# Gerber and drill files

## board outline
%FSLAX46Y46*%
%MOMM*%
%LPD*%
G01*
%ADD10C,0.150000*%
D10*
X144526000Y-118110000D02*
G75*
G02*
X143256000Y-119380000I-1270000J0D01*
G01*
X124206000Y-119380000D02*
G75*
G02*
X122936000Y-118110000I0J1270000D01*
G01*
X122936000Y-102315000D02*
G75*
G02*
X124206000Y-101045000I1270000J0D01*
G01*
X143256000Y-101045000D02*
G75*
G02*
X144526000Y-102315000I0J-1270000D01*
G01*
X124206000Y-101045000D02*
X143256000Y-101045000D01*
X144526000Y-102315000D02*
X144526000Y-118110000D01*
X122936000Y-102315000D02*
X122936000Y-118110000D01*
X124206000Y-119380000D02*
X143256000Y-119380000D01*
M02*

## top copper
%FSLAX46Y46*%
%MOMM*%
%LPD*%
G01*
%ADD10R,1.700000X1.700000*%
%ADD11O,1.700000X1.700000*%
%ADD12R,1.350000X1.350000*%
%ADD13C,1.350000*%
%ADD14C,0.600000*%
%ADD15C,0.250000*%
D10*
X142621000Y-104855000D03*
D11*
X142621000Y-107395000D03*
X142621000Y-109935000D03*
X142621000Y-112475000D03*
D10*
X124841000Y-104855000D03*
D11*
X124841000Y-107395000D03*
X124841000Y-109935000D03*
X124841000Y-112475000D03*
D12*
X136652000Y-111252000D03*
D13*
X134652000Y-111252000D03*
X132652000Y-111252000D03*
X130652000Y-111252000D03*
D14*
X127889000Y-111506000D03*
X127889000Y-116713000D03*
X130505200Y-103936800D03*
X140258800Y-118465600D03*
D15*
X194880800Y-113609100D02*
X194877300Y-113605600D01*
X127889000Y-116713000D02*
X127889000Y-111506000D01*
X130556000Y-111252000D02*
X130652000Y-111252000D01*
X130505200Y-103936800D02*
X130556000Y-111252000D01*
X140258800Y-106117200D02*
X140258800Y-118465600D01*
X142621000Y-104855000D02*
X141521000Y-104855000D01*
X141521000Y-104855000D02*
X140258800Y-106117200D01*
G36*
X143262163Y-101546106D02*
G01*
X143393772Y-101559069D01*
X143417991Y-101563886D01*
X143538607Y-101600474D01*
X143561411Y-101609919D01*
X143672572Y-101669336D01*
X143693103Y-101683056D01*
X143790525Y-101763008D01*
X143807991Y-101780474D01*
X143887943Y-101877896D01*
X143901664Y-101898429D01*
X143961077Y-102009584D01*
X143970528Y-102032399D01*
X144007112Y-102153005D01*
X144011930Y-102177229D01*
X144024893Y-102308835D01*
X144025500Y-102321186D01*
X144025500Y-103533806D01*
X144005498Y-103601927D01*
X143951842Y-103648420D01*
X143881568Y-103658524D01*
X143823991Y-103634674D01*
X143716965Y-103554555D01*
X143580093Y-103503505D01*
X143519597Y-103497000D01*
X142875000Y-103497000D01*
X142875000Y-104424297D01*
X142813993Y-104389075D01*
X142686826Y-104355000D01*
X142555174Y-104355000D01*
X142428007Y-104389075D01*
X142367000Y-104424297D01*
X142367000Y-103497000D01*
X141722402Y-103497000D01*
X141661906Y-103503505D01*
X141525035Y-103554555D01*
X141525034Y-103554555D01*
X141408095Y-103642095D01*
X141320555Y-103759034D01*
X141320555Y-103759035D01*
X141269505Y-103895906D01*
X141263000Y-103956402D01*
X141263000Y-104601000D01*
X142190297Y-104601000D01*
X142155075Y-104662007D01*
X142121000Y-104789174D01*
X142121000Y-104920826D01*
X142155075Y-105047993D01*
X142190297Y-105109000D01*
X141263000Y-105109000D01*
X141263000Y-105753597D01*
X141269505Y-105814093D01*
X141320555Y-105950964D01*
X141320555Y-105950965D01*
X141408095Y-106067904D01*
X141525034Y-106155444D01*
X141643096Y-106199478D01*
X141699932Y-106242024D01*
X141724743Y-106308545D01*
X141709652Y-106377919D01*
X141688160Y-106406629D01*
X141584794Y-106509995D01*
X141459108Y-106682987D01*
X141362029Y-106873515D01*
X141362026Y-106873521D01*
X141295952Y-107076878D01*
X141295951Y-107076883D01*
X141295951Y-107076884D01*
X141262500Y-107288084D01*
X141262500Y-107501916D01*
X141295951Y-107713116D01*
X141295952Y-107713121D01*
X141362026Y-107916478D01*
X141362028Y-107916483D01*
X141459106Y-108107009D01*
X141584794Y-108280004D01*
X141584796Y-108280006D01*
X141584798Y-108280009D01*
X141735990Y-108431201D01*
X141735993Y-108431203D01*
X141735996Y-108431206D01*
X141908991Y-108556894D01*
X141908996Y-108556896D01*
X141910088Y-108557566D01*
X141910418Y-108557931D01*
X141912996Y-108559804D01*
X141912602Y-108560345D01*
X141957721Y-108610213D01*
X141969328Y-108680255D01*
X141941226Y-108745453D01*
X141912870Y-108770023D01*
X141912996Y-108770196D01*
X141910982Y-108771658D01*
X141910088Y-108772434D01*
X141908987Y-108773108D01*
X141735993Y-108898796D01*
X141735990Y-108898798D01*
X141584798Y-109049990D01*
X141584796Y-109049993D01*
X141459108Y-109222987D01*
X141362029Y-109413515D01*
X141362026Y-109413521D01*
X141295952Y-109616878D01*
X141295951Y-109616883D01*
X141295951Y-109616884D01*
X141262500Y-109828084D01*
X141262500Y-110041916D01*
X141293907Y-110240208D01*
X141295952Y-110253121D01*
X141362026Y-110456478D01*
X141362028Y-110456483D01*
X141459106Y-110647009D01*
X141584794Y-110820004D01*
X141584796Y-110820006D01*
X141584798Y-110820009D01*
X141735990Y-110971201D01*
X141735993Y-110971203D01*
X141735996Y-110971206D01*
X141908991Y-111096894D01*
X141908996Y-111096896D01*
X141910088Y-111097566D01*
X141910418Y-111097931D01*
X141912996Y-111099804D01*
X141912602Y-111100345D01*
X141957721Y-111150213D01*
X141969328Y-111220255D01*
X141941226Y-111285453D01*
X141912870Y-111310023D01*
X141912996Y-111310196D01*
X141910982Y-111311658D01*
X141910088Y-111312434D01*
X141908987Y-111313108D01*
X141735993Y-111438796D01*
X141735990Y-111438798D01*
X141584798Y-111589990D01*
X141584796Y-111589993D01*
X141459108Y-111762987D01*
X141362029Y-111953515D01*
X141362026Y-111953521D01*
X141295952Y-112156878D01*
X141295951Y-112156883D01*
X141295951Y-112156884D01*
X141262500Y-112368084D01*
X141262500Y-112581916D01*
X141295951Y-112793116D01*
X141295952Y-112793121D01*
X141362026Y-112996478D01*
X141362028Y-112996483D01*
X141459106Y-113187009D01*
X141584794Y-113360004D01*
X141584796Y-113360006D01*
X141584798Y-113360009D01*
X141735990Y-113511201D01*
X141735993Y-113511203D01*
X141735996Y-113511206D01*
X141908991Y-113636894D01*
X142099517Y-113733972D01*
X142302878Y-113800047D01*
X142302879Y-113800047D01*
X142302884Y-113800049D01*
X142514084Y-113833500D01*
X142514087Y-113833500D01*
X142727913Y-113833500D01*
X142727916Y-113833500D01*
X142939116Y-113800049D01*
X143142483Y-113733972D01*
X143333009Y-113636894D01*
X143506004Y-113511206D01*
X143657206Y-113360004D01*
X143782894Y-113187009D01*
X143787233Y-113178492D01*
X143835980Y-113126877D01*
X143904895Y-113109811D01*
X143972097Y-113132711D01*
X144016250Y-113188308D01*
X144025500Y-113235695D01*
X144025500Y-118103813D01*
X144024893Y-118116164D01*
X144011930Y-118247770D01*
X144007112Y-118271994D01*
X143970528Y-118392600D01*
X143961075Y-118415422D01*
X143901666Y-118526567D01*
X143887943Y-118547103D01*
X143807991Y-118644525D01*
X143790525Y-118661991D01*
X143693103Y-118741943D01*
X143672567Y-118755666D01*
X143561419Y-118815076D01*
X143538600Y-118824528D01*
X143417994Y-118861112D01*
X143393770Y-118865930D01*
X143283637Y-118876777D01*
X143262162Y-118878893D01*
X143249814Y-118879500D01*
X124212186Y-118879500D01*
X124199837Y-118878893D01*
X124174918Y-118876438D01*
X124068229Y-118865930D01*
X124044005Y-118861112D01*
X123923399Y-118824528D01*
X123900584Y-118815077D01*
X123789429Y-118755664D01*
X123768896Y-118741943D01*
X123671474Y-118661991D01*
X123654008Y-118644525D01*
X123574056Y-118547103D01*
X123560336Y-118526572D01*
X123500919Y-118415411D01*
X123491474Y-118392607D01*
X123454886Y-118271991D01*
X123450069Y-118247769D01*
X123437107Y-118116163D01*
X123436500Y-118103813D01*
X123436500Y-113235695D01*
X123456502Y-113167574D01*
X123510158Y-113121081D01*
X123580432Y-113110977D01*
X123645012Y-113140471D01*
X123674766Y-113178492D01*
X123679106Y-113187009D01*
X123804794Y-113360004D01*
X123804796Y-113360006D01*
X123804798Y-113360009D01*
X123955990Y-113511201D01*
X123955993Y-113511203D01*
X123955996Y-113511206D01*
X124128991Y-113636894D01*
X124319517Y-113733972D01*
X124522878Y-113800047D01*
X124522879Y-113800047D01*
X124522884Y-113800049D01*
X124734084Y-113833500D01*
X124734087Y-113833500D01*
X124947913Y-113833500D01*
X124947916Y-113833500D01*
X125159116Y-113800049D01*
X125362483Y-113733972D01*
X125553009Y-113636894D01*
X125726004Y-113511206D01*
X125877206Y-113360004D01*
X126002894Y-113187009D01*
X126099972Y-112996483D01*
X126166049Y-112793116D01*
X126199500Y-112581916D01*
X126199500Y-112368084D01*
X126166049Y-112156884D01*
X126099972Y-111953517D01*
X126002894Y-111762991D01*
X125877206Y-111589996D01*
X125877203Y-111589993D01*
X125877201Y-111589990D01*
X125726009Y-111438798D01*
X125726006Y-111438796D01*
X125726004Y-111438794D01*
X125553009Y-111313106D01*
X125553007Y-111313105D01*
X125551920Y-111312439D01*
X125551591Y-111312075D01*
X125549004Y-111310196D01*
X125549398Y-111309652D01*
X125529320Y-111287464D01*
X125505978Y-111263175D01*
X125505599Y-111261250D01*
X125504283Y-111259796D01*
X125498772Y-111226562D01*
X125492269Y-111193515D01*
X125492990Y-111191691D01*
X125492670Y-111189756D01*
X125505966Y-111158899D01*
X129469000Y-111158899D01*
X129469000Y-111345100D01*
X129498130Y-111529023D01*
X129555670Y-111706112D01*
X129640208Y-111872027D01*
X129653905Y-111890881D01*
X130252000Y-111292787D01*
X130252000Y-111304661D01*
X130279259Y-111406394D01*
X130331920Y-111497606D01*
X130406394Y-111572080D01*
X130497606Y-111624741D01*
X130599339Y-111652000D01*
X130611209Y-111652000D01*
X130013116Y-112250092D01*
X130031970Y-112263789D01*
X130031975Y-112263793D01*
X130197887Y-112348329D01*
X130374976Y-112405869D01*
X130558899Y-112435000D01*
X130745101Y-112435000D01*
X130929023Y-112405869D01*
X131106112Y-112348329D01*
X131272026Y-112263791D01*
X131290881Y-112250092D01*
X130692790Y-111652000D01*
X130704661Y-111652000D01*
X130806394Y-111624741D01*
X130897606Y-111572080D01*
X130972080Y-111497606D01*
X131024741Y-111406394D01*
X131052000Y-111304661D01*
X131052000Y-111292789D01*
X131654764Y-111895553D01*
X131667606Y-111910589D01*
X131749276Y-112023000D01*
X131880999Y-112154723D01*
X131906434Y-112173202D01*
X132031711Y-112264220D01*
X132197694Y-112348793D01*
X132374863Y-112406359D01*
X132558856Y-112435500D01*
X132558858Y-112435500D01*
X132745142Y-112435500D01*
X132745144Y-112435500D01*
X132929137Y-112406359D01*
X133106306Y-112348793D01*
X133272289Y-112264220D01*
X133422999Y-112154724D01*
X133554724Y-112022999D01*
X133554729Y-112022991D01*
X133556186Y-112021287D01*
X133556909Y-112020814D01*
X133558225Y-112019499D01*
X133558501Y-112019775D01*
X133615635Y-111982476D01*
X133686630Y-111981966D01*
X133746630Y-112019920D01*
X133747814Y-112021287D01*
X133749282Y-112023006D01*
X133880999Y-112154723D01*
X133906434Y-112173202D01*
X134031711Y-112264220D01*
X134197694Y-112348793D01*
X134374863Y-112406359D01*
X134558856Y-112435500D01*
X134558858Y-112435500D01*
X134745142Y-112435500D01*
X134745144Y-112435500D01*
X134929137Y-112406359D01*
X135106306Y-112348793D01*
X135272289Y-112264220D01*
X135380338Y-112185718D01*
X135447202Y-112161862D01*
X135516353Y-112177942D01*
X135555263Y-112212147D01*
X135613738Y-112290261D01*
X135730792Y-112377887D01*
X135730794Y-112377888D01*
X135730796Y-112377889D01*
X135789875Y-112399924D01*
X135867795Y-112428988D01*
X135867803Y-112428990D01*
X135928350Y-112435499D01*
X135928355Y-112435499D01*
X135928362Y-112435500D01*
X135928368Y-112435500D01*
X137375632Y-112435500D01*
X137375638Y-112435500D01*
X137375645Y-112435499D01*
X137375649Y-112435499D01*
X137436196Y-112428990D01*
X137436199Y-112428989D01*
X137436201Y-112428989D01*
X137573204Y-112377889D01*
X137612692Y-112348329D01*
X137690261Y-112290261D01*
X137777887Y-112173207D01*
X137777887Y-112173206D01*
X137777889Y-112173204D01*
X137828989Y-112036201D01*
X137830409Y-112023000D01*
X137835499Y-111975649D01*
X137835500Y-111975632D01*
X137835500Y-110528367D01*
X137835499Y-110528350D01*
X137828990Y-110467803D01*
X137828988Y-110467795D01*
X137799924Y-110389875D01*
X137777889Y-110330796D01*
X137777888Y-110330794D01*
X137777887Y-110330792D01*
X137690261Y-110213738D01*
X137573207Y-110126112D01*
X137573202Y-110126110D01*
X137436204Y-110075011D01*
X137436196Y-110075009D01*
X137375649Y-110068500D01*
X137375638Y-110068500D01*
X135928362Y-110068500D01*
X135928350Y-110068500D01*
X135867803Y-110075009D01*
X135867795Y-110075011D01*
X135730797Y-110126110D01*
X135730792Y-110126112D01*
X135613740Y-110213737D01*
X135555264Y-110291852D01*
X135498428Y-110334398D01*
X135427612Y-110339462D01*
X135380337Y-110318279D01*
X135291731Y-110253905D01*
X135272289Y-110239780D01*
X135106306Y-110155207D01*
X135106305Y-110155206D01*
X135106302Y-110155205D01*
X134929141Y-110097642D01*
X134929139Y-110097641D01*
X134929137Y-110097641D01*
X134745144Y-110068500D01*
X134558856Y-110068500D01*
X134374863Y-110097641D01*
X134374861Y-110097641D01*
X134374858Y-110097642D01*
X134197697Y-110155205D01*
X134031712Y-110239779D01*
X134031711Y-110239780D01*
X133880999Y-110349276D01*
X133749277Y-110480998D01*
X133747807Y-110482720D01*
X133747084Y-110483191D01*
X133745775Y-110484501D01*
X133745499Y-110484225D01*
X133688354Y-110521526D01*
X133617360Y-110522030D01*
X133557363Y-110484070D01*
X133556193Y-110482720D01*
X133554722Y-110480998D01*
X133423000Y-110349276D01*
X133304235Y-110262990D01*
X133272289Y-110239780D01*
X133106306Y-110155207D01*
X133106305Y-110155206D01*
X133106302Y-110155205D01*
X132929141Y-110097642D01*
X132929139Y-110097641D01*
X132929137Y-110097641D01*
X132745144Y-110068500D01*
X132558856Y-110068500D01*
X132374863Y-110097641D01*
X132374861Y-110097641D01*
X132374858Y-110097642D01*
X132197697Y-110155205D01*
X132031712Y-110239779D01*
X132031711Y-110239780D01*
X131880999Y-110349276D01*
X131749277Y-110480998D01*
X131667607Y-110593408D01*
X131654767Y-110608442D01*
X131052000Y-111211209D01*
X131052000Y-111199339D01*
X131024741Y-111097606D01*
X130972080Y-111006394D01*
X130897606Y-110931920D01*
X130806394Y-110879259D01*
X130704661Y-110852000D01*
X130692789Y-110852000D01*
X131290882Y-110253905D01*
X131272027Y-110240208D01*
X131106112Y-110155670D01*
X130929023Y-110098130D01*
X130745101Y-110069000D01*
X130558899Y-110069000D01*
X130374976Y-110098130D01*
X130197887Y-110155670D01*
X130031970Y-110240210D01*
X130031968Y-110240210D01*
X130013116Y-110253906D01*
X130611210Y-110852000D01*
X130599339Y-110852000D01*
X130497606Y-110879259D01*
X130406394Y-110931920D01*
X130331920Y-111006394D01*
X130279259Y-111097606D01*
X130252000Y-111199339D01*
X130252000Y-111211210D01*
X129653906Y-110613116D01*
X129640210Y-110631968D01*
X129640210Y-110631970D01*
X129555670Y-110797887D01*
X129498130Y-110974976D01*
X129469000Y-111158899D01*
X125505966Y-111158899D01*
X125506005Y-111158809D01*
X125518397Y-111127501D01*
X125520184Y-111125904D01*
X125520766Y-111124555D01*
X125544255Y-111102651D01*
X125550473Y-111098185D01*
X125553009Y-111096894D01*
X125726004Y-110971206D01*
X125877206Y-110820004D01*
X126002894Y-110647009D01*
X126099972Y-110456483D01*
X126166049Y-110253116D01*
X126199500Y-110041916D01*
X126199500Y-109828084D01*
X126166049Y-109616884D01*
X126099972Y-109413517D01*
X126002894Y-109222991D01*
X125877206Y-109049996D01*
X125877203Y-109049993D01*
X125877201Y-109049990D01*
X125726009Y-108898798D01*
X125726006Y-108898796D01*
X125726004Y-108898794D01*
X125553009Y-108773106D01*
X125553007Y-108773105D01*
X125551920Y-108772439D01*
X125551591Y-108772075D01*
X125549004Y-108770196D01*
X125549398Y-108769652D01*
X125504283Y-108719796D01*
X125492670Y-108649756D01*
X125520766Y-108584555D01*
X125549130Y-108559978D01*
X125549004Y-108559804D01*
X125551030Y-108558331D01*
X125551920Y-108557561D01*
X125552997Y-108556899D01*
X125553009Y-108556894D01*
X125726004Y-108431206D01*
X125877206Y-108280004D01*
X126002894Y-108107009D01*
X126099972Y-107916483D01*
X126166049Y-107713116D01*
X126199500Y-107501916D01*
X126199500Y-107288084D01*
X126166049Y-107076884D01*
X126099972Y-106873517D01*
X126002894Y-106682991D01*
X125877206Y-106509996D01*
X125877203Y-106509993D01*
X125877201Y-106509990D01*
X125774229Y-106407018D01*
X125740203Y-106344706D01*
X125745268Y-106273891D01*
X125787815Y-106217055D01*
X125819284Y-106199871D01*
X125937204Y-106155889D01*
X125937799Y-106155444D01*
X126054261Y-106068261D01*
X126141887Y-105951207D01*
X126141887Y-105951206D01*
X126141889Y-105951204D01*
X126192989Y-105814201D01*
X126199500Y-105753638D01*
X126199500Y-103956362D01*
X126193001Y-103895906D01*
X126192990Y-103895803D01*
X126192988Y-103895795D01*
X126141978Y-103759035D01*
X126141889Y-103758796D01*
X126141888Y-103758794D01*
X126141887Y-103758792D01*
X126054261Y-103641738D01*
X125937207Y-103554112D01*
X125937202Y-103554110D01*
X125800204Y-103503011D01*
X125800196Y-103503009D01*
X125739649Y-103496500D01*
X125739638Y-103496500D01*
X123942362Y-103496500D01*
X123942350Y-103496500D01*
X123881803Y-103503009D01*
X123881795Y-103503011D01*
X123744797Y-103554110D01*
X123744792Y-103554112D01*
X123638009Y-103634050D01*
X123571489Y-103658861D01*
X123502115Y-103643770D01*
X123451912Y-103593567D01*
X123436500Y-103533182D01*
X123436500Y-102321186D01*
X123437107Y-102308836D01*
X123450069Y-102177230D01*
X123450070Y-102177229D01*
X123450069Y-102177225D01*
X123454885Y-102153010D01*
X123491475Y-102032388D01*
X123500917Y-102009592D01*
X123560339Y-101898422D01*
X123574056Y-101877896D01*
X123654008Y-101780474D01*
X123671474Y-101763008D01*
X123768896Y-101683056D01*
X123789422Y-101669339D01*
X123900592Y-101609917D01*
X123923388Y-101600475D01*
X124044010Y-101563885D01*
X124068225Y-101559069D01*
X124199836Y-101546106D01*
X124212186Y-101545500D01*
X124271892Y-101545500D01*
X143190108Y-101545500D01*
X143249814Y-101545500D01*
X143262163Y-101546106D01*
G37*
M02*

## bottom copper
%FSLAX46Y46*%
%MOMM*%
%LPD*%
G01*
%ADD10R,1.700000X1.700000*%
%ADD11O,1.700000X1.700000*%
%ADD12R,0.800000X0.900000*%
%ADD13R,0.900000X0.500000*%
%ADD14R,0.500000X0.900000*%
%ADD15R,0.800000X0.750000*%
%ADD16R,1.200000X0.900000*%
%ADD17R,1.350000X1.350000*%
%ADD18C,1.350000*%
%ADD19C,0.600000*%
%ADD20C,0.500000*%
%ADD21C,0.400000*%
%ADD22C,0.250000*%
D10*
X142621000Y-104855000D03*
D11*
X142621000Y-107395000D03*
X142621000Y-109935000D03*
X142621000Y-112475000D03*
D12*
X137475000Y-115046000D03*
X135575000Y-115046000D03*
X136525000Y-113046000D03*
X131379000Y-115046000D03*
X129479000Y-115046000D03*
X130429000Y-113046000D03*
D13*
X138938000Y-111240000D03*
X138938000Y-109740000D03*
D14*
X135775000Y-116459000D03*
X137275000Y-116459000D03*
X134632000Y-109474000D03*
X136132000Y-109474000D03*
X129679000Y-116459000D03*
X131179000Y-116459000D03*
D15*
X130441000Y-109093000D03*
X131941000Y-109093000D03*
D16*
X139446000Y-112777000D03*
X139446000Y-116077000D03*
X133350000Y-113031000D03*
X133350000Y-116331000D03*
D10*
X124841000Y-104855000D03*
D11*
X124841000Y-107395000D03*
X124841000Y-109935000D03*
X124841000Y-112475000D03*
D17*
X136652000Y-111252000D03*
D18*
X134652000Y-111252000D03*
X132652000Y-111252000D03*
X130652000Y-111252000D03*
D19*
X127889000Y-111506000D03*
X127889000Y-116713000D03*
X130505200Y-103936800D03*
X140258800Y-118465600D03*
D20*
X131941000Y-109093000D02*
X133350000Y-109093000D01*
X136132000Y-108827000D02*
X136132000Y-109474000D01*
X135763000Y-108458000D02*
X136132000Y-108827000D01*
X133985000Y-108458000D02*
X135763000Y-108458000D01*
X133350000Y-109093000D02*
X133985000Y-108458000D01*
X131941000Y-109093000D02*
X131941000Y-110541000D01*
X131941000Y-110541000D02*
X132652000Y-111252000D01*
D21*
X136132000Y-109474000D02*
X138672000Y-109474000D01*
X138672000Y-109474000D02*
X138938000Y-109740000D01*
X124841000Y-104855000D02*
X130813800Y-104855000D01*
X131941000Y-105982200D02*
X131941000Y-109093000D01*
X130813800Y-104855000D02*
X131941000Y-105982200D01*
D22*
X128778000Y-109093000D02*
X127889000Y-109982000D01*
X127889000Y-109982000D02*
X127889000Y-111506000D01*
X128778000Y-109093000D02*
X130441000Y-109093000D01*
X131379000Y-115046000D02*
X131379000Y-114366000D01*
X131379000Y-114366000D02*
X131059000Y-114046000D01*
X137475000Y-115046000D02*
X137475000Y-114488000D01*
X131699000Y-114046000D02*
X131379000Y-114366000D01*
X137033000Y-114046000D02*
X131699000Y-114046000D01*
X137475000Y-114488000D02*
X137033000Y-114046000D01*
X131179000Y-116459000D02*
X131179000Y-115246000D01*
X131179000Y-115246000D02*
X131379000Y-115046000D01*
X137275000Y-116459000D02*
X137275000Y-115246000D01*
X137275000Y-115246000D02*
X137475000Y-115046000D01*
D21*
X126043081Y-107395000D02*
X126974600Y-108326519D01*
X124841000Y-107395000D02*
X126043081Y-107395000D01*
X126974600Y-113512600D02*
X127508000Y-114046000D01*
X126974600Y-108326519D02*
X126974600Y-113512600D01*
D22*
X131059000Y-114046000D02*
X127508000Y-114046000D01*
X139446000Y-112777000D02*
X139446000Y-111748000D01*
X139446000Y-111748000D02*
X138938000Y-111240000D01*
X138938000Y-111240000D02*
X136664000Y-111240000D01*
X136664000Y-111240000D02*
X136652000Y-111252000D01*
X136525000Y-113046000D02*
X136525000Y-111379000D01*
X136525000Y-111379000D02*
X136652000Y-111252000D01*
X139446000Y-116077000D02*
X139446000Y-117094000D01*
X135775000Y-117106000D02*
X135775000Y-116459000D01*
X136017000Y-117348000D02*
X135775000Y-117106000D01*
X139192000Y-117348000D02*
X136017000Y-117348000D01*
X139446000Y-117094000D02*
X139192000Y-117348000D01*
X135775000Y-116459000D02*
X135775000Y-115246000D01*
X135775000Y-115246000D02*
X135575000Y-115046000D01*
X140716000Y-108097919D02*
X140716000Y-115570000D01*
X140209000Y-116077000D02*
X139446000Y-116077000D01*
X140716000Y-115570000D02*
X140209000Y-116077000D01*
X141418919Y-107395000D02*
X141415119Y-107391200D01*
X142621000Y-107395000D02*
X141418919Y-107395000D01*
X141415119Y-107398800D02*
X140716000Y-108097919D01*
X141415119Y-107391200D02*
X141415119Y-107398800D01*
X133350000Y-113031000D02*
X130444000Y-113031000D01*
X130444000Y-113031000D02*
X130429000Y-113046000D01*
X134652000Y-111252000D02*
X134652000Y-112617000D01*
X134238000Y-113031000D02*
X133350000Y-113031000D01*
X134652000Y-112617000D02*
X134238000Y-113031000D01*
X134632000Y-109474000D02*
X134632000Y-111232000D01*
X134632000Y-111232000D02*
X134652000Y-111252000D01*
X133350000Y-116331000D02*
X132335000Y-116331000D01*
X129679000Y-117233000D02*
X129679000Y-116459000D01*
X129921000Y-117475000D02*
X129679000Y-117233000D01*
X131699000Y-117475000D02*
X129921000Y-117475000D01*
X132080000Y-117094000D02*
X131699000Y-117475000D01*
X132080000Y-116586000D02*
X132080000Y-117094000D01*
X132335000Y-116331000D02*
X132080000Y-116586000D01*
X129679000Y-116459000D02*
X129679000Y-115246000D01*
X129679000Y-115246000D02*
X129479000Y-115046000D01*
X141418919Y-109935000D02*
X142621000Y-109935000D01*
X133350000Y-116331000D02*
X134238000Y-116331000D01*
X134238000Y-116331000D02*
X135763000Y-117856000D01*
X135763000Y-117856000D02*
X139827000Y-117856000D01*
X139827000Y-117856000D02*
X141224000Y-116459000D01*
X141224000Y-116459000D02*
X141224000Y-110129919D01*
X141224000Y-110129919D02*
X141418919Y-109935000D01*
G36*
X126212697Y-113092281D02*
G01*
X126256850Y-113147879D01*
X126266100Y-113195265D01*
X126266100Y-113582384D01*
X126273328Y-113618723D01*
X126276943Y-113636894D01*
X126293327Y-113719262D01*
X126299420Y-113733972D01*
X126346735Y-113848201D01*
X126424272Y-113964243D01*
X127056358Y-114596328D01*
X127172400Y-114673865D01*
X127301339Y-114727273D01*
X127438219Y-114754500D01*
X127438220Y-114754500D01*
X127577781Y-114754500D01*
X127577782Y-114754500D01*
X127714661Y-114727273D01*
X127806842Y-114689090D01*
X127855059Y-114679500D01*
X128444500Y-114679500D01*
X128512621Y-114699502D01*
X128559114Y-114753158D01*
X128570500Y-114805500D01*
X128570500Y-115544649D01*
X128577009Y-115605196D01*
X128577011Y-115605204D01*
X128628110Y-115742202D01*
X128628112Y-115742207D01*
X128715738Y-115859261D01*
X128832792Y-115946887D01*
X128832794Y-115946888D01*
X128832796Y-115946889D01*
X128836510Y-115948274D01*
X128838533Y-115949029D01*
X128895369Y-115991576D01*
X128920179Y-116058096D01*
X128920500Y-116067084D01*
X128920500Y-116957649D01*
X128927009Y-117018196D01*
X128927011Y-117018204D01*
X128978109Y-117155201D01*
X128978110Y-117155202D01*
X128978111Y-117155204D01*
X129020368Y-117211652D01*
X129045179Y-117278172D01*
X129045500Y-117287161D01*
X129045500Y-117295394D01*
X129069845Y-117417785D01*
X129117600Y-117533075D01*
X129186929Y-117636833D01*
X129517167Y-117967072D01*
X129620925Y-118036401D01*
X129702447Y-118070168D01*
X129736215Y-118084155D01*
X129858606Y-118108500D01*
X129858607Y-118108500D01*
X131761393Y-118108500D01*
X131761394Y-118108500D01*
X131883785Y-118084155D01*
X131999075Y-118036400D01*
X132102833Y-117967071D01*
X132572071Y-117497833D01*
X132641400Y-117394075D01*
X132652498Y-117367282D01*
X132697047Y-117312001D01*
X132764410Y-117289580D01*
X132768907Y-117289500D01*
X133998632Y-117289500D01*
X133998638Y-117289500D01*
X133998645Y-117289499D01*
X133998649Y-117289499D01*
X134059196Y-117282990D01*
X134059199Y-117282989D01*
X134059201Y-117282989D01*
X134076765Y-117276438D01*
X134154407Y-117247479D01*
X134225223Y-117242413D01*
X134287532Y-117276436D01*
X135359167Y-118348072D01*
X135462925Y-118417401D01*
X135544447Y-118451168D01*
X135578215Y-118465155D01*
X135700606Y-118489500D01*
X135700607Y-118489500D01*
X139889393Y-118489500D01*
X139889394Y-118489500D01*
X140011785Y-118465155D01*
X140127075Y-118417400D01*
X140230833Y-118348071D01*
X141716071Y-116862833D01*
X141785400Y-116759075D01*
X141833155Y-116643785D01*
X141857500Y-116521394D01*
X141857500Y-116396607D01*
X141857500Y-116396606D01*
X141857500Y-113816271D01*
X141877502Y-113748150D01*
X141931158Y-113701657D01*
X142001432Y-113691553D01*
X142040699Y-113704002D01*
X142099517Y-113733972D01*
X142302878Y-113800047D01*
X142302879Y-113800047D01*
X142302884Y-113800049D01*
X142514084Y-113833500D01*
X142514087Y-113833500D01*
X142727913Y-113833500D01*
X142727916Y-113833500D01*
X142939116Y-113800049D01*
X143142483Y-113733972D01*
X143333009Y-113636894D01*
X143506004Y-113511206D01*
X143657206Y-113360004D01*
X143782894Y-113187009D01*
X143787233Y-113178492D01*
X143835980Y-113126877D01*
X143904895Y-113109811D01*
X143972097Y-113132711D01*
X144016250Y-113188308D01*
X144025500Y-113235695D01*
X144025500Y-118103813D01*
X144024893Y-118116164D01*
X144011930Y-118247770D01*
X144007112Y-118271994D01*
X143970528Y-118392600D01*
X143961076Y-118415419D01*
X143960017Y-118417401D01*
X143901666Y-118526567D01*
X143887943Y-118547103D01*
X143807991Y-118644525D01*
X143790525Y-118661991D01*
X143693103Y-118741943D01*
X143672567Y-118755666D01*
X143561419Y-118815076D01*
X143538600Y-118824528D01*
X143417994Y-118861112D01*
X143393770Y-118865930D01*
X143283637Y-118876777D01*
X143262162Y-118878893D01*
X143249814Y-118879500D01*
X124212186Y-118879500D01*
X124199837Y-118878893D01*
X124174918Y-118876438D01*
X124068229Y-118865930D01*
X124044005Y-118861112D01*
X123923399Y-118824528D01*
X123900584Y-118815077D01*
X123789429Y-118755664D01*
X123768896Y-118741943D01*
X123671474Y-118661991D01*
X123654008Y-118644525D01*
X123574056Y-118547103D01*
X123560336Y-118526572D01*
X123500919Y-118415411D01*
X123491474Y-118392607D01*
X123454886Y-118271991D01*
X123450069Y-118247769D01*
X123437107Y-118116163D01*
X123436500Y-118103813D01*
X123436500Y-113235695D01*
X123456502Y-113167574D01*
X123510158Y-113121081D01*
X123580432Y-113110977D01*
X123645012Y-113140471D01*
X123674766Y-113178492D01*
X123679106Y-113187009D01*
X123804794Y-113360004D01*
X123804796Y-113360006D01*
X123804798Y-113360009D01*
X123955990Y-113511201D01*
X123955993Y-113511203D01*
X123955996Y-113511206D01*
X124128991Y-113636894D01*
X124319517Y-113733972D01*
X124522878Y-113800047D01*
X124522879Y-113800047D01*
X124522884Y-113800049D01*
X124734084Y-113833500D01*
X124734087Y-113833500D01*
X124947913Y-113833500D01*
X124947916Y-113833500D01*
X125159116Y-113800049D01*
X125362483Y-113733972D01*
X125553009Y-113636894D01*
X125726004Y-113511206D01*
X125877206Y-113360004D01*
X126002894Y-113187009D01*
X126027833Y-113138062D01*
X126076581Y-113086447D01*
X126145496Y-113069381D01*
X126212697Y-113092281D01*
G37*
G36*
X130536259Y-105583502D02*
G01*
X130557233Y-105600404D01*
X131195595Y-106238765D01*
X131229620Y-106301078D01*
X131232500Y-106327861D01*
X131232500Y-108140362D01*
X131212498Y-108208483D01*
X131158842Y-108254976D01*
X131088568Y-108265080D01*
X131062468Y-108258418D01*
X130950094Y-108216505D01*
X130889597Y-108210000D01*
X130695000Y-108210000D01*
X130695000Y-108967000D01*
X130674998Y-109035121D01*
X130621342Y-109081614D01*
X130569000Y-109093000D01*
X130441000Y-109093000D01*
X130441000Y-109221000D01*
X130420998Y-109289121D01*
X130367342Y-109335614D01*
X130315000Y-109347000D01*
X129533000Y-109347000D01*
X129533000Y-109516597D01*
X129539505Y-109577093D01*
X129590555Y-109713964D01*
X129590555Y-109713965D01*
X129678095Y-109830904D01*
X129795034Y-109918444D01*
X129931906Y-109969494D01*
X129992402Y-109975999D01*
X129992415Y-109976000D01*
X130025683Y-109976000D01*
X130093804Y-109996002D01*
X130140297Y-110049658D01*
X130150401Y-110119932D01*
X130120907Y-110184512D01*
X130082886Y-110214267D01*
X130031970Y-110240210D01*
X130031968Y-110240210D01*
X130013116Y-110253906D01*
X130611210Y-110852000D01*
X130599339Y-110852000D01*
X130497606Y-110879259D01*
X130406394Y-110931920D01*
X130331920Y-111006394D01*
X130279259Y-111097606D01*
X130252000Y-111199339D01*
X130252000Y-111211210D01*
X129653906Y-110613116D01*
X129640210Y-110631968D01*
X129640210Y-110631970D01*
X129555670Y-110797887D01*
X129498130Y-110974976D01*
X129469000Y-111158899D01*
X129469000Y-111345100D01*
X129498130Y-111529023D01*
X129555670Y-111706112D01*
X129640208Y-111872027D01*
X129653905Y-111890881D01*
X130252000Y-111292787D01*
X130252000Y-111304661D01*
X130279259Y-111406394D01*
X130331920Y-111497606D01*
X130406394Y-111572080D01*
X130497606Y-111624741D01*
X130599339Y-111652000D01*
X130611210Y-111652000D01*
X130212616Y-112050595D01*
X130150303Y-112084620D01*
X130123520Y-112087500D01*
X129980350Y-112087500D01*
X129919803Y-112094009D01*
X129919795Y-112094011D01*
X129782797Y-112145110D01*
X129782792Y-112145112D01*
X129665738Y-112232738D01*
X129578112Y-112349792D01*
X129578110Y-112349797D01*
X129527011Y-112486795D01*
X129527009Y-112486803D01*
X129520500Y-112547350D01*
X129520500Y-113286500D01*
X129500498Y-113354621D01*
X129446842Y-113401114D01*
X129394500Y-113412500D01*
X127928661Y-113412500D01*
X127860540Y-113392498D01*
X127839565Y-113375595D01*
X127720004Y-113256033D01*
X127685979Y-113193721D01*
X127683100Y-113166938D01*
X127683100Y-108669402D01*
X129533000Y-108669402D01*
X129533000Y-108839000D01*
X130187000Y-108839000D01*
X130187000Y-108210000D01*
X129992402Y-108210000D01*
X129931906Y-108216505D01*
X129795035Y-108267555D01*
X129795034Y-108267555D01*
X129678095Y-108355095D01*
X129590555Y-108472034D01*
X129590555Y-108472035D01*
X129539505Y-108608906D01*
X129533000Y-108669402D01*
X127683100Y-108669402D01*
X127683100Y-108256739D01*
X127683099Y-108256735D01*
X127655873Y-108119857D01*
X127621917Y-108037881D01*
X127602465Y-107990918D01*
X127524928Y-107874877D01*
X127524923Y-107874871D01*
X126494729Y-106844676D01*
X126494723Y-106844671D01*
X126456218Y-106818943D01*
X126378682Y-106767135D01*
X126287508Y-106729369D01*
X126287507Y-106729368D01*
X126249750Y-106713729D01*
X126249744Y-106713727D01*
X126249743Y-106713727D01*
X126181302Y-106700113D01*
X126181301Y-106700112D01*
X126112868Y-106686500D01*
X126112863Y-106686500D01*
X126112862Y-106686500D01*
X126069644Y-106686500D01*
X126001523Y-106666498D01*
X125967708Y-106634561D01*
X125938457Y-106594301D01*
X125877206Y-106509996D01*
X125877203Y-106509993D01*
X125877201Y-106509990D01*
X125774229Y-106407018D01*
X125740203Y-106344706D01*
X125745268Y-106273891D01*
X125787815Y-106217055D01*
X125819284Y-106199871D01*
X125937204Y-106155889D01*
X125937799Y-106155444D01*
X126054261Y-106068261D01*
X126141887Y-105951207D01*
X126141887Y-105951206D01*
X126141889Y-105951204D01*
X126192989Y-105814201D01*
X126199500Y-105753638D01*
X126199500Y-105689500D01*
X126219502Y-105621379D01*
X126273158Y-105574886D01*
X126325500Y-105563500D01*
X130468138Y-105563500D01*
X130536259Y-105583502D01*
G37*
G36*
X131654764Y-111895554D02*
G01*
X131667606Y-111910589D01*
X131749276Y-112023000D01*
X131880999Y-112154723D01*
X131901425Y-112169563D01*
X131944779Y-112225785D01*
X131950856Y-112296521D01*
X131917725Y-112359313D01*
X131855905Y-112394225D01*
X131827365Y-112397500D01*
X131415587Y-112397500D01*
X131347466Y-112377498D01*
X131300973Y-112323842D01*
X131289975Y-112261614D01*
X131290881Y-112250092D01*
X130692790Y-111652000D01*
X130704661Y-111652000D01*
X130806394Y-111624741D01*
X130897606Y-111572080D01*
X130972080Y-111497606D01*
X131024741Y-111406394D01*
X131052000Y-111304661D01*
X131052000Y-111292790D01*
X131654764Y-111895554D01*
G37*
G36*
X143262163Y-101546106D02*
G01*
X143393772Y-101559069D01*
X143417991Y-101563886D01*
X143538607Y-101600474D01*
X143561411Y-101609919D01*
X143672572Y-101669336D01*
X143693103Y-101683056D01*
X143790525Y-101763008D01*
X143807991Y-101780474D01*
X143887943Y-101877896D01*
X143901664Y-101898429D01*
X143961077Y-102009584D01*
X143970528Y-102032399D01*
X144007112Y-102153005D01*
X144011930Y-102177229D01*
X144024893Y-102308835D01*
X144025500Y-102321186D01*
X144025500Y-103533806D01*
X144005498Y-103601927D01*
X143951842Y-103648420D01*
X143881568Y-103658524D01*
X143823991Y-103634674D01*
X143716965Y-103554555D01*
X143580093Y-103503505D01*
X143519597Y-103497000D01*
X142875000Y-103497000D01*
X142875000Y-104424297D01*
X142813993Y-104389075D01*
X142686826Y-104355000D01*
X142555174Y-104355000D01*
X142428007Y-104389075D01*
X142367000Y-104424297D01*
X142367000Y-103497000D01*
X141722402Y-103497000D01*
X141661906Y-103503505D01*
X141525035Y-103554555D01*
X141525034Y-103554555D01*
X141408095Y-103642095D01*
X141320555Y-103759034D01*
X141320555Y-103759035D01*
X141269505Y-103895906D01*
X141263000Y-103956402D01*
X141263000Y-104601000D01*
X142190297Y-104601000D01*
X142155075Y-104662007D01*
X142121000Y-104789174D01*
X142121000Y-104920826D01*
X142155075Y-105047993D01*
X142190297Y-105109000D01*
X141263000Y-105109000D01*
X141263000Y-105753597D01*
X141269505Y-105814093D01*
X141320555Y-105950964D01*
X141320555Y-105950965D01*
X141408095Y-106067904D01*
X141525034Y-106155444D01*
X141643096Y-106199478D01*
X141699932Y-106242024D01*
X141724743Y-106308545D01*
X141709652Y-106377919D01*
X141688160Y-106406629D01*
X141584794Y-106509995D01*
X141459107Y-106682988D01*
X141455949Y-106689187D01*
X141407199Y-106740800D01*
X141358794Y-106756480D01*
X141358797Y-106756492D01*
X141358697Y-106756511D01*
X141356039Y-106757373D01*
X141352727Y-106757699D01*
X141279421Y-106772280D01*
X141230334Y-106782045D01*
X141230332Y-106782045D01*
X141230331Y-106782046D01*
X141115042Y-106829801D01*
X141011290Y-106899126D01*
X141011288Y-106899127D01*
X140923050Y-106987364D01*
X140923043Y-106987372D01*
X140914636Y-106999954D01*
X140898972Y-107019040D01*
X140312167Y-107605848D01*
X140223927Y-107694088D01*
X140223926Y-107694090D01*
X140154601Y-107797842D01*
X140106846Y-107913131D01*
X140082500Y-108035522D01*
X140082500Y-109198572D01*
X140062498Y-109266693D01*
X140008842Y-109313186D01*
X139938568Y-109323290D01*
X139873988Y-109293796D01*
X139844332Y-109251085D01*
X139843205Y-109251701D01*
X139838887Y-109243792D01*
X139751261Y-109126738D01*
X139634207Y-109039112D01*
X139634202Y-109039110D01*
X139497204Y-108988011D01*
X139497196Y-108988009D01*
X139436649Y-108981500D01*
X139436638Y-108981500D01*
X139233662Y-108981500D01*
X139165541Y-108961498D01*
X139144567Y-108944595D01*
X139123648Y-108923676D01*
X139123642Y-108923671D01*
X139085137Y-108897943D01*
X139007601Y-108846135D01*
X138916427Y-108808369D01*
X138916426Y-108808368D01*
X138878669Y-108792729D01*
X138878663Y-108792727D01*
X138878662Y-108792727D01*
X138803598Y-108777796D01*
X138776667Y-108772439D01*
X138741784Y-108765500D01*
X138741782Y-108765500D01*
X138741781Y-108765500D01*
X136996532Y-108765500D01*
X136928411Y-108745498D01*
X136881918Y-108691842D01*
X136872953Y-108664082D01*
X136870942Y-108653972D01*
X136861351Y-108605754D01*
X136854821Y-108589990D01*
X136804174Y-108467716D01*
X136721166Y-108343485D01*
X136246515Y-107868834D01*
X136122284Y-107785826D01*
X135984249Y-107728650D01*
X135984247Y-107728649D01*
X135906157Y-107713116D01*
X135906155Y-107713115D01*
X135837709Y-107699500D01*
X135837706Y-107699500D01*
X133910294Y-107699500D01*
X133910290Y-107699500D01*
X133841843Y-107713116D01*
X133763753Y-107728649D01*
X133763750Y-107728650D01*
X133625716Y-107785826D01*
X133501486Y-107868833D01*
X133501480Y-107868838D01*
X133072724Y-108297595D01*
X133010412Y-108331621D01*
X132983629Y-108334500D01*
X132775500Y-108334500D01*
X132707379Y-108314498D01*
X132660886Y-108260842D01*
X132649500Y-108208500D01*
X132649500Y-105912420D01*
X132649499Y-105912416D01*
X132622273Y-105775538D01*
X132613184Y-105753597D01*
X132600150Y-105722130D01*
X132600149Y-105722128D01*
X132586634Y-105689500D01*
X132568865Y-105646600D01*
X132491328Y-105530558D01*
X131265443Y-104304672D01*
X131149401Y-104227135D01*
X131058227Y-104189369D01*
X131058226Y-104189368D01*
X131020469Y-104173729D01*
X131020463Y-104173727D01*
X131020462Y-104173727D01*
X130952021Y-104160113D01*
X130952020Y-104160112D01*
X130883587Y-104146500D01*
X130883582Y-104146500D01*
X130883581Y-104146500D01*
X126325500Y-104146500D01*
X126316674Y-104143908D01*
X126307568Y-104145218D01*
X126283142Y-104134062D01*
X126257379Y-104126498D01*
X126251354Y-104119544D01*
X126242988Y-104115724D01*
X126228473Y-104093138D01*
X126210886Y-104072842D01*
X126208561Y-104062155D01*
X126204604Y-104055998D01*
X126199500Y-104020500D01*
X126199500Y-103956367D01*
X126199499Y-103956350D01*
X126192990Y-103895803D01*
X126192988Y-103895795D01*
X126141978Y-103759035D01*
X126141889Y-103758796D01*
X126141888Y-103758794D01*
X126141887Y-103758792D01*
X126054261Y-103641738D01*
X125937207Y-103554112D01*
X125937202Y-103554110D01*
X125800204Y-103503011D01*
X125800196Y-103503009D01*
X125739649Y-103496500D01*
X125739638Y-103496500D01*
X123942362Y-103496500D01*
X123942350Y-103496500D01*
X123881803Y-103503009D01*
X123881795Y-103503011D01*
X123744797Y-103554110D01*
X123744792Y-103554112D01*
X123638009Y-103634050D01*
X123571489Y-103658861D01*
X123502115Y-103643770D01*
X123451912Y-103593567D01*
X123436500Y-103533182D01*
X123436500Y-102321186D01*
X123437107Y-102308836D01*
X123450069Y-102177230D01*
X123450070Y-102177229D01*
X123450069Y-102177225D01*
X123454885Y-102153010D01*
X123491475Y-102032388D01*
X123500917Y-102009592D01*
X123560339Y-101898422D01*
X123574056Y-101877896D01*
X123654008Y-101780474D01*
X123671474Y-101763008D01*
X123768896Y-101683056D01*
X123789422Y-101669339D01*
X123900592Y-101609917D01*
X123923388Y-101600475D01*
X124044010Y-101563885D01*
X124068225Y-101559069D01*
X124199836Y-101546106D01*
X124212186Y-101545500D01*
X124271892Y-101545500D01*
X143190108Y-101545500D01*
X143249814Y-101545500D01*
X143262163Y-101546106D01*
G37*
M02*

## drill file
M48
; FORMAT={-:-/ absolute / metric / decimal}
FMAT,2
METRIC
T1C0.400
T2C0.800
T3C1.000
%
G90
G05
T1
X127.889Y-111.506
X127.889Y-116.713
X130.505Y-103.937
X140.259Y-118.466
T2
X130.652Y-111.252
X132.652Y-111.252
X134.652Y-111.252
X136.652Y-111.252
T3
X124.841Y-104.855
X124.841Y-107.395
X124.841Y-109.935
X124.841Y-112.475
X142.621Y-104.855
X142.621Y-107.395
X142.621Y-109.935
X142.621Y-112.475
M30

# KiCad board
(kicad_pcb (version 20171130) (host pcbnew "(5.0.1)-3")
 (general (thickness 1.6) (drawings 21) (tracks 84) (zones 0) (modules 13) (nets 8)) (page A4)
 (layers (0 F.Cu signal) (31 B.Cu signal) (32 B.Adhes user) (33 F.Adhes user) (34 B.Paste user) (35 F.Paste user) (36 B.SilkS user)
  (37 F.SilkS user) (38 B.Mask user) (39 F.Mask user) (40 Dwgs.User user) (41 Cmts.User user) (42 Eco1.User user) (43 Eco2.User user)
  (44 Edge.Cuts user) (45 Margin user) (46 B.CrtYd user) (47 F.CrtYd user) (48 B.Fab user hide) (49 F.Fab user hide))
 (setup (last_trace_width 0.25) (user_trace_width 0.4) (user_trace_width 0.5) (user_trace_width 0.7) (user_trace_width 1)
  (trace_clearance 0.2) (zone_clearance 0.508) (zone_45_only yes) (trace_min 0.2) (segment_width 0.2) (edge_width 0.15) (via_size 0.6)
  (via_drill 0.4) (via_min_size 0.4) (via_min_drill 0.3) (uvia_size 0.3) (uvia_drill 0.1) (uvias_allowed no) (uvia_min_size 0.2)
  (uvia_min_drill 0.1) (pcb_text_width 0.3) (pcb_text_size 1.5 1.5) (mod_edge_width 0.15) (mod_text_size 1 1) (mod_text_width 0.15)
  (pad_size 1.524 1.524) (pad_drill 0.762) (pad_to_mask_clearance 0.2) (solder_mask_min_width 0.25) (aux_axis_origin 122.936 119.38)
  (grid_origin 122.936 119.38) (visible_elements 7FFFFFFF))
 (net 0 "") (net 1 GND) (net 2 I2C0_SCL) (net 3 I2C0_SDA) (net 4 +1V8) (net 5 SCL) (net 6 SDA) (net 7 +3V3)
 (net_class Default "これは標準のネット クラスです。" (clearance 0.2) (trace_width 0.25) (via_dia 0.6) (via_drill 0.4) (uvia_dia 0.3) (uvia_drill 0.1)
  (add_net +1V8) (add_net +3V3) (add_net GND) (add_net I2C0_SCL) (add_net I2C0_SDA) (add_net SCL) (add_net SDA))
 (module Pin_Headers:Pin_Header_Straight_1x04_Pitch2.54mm (layer F.Cu) (at 142.621 104.855)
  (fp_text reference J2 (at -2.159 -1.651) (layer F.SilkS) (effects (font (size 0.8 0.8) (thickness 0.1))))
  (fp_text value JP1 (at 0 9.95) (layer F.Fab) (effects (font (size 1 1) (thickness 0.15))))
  (pad 1 thru_hole rect (at 0 0) (size 1.7 1.7) (drill 1) (layers *.Cu *.Mask) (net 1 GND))
  (pad 2 thru_hole oval (at 0 2.54) (size 1.7 1.7) (drill 1) (layers *.Cu *.Mask) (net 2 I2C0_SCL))
  (pad 3 thru_hole oval (at 0 5.08) (size 1.7 1.7) (drill 1) (layers *.Cu *.Mask) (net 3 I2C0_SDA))
  (pad 4 thru_hole oval (at 0 7.62) (size 1.7 1.7) (drill 1) (layers *.Cu *.Mask)))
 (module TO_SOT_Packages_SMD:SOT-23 (layer B.Cu) (at 136.525 114.046 90)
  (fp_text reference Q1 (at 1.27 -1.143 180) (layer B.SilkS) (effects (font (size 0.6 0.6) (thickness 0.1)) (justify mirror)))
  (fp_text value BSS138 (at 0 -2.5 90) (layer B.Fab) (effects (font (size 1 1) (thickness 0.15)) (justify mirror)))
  (pad 1 smd rect (at -1 0.95 90) (size 0.9 0.8) (layers B.Cu B.Paste B.Mask) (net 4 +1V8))
  (pad 2 smd rect (at -1 -0.95 90) (size 0.9 0.8) (layers B.Cu B.Paste B.Mask) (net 2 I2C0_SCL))
  (pad 3 smd rect (at 1 0 90) (size 0.9 0.8) (layers B.Cu B.Paste B.Mask) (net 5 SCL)))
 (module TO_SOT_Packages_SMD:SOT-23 (layer B.Cu) (at 130.429 114.046 90)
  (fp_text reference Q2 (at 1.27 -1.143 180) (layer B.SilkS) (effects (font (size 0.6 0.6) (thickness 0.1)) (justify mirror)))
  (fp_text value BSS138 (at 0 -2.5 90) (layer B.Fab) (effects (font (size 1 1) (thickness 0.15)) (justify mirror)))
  (pad 1 smd rect (at -1 0.95 90) (size 0.9 0.8) (layers B.Cu B.Paste B.Mask) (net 4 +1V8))
  (pad 2 smd rect (at -1 -0.95 90) (size 0.9 0.8) (layers B.Cu B.Paste B.Mask) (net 3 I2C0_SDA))
  (pad 3 smd rect (at 1 0 90) (size 0.9 0.8) (layers B.Cu B.Paste B.Mask) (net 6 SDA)))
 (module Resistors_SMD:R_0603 (layer B.Cu) (at 138.938 110.49 90)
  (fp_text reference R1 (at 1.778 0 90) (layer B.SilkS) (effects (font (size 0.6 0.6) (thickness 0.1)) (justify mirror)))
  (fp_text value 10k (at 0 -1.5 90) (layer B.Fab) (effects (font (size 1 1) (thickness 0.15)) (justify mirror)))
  (pad 1 smd rect (at -0.75 0 90) (size 0.5 0.9) (layers B.Cu B.Paste B.Mask) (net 5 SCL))
  (pad 2 smd rect (at 0.75 0 90) (size 0.5 0.9) (layers B.Cu B.Paste B.Mask) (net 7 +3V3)))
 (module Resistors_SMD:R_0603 (layer B.Cu) (at 136.525 116.459)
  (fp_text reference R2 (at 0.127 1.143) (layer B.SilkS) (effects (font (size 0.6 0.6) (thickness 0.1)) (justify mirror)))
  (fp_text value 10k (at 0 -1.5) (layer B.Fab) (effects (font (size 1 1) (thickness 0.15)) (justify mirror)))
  (pad 1 smd rect (at -0.75 0) (size 0.5 0.9) (layers B.Cu B.Paste B.Mask) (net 2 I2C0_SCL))
  (pad 2 smd rect (at 0.75 0) (size 0.5 0.9) (layers B.Cu B.Paste B.Mask) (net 4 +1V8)))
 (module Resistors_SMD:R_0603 (layer B.Cu) (at 135.382 109.474)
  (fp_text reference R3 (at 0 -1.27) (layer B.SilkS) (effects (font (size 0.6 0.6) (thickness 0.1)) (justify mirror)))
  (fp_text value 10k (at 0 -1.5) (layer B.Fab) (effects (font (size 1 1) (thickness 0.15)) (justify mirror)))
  (pad 1 smd rect (at -0.75 0) (size 0.5 0.9) (layers B.Cu B.Paste B.Mask) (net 6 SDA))
  (pad 2 smd rect (at 0.75 0) (size 0.5 0.9) (layers B.Cu B.Paste B.Mask) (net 7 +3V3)))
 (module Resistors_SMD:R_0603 (layer B.Cu) (at 130.429 116.459)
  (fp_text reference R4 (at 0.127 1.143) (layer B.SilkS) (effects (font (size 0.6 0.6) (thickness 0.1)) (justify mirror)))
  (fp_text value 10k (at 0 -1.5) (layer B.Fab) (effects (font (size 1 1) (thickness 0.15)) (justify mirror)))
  (pad 1 smd rect (at -0.75 0) (size 0.5 0.9) (layers B.Cu B.Paste B.Mask) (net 3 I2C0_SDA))
  (pad 2 smd rect (at 0.75 0) (size 0.5 0.9) (layers B.Cu B.Paste B.Mask) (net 4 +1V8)))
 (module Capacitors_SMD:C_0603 (layer B.Cu) (at 131.191 109.093 180)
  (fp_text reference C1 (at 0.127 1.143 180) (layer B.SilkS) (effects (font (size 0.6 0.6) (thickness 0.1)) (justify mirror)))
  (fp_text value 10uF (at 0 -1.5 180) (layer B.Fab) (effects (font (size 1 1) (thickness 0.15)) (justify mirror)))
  (pad 2 smd rect (at 0.75 0 180) (size 0.8 0.75) (layers B.Cu B.Paste B.Mask) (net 1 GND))
  (pad 1 smd rect (at -0.75 0 180) (size 0.8 0.75) (layers B.Cu B.Paste B.Mask) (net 7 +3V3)))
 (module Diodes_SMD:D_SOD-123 (layer B.Cu) (at 139.446 114.427 270)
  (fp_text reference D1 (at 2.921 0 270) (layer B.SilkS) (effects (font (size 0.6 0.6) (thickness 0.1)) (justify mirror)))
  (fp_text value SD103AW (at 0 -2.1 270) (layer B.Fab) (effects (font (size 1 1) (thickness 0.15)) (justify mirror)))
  (pad 1 smd rect (at -1.65 0 270) (size 0.9 1.2) (layers B.Cu B.Paste B.Mask) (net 5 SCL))
  (pad 2 smd rect (at 1.65 0 270) (size 0.9 1.2) (layers B.Cu B.Paste B.Mask) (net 2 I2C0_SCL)))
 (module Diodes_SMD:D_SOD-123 (layer B.Cu) (at 133.35 114.681 270)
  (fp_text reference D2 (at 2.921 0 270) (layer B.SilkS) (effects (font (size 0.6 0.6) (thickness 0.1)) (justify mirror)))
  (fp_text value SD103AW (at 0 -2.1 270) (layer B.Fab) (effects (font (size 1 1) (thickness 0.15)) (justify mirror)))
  (pad 1 smd rect (at -1.65 0 270) (size 0.9 1.2) (layers B.Cu B.Paste B.Mask) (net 6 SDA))
  (pad 2 smd rect (at 1.65 0 270) (size 0.9 1.2) (layers B.Cu B.Paste B.Mask) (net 3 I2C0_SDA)))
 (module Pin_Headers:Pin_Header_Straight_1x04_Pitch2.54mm (layer F.Cu) (at 124.841 104.855)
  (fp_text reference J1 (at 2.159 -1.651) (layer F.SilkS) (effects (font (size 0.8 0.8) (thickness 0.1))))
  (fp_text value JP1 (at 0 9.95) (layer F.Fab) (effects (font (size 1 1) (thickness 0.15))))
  (pad 1 thru_hole rect (at 0 0) (size 1.7 1.7) (drill 1) (layers *.Cu *.Mask) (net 7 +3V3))
  (pad 2 thru_hole oval (at 0 2.54) (size 1.7 1.7) (drill 1) (layers *.Cu *.Mask) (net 4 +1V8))
  (pad 3 thru_hole oval (at 0 5.08) (size 1.7 1.7) (drill 1) (layers *.Cu *.Mask))
  (pad 4 thru_hole oval (at 0 7.62) (size 1.7 1.7) (drill 1) (layers *.Cu *.Mask)))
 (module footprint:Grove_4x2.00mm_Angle (layer F.Cu) (at 136.652 111.252 180)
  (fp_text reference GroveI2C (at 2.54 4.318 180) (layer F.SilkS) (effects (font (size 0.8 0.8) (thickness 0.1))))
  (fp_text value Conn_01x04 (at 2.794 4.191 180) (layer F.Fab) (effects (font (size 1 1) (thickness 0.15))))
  (pad 1 thru_hole rect (at 0 0 180) (size 1.35 1.35) (drill 0.8) (layers *.Cu *.Mask) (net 5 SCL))
  (pad 2 thru_hole circle (at 2 0 180) (size 1.35 1.35) (drill 0.8) (layers *.Cu *.Mask) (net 6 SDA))
  (pad 3 thru_hole circle (at 4 0 180) (size 1.35 1.35) (drill 0.8) (layers *.Cu *.Mask) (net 7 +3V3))
  (pad 4 thru_hole circle (at 6 0 180) (size 1.35 1.35) (drill 0.8) (layers *.Cu *.Mask) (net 1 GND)))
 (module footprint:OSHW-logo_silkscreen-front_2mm (layer F.Cu) (at 127.508 118.11)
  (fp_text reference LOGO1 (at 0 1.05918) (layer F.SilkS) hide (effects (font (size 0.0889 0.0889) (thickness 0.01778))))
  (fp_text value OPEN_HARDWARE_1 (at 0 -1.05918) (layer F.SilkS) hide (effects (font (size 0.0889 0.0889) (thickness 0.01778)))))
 (gr_arc (start 143.256 118.11) (end 144.526 118.11) (angle 90) (layer Edge.Cuts) (width 0.15))
 (gr_arc (start 124.206 118.11) (end 124.206 119.38) (angle 90) (layer Edge.Cuts) (width 0.15))
 (gr_arc (start 124.206 102.315) (end 122.936 102.315) (angle 90) (layer Edge.Cuts) (width 0.15))
 (gr_arc (start 143.256 102.315) (end 143.256 101.045) (angle 90) (layer Edge.Cuts) (width 0.15))
 (gr_line (start 124.206 101.045) (end 143.256 101.045) (angle 90) (layer Edge.Cuts) (width 0.15))
 (gr_line (start 144.526 102.315) (end 144.526 118.11) (angle 90) (layer Edge.Cuts) (width 0.15))
 (gr_line (start 122.936 102.315) (end 122.936 118.11) (angle 90) (layer Edge.Cuts) (width 0.15))
 (gr_line (start 124.206 119.38) (end 143.256 119.38) (angle 90) (layer Edge.Cuts) (width 0.15))
 (segment (start 194.8808 113.6091) (end 194.8773 113.6056) (width 0.25) (layer F.Cu) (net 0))
 (segment (start 131.941 109.093) (end 133.35 109.093) (width 0.5) (layer B.Cu) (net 7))
 (segment (start 136.132 108.827) (end 136.132 109.474) (width 0.5) (layer B.Cu) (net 7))
 (segment (start 135.763 108.458) (end 136.132 108.827) (width 0.5) (layer B.Cu) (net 7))
 (segment (start 133.985 108.458) (end 135.763 108.458) (width 0.5) (layer B.Cu) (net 7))
 (segment (start 133.35 109.093) (end 133.985 108.458) (width 0.5) (layer B.Cu) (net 7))
 (segment (start 131.941 109.093) (end 131.941 110.541) (width 0.5) (layer B.Cu) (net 7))
 (segment (start 131.941 110.541) (end 132.652 111.252) (width 0.5) (layer B.Cu) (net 7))
 (segment (start 136.132 109.474) (end 138.672 109.474) (width 0.4) (layer B.Cu) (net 7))
 (segment (start 138.672 109.474) (end 138.938 109.74) (width 0.4) (layer B.Cu) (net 7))
 (segment (start 124.841 104.855) (end 130.8138 104.855) (width 0.4) (layer B.Cu) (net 7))
 (segment (start 131.941 105.9822) (end 131.941 109.093) (width 0.4) (layer B.Cu) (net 7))
 (segment (start 130.8138 104.855) (end 131.941 105.9822) (width 0.4) (layer B.Cu) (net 7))
 (segment (start 127.889 116.713) (end 127.889 111.506) (width 0.25) (layer F.Cu) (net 1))
 (segment (start 128.778 109.093) (end 127.889 109.982) (width 0.25) (layer B.Cu) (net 1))
 (segment (start 127.889 109.982) (end 127.889 111.506) (width 0.25) (layer B.Cu) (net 1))
 (via (at 127.889 111.506) (size 0.6) (drill 0.4) (layers F.Cu B.Cu) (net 1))
 (segment (start 128.778 109.093) (end 130.441 109.093) (width 0.25) (layer B.Cu) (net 1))
 (via (at 127.889 116.713) (size 0.6) (drill 0.4) (layers F.Cu B.Cu) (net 1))
 (via (at 130.5052 103.9368) (size 0.6) (drill 0.4) (layers F.Cu B.Cu) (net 1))
 (segment (start 130.556 111.252) (end 130.652 111.252) (width 0.25) (layer F.Cu) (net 1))
 (segment (start 130.5052 103.9368) (end 130.556 111.252) (width 0.25) (layer F.Cu) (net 1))
 (via (at 140.2588 118.4656) (size 0.6) (drill 0.4) (layers F.Cu B.Cu) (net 1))
 (segment (start 140.2588 106.1172) (end 140.2588 118.4656) (width 0.25) (layer F.Cu) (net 1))
 (segment (start 142.621 104.855) (end 141.521 104.855) (width 0.25) (layer F.Cu) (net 1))
 (segment (start 141.521 104.855) (end 140.2588 106.1172) (width 0.25) (layer F.Cu) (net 1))
 (segment (start 131.379 115.046) (end 131.379 114.366) (width 0.25) (layer B.Cu) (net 4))
 (segment (start 131.379 114.366) (end 131.059 114.046) (width 0.25) (layer B.Cu) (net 4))
 (segment (start 137.475 115.046) (end 137.475 114.488) (width 0.25) (layer B.Cu) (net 4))
 (segment (start 131.699 114.046) (end 131.379 114.366) (width 0.25) (layer B.Cu) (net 4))
 (segment (start 137.033 114.046) (end 131.699 114.046) (width 0.25) (layer B.Cu) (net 4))
 (segment (start 137.475 114.488) (end 137.033 114.046) (width 0.25) (layer B.Cu) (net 4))
 (segment (start 131.179 116.459) (end 131.179 115.246) (width 0.25) (layer B.Cu) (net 4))
 (segment (start 131.179 115.246) (end 131.379 115.046) (width 0.25) (layer B.Cu) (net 4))
 (segment (start 137.275 116.459) (end 137.275 115.246) (width 0.25) (layer B.Cu) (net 4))
 (segment (start 137.275 115.246) (end 137.475 115.046) (width 0.25) (layer B.Cu) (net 4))
 (segment (start 126.043081 107.395) (end 126.9746 108.326519) (width 0.4) (layer B.Cu) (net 4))
 (segment (start 124.841 107.395) (end 126.043081 107.395) (width 0.4) (layer B.Cu) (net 4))
 (segment (start 126.9746 113.5126) (end 127.508 114.046) (width 0.4) (layer B.Cu) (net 4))
 (segment (start 126.9746 108.326519) (end 126.9746 113.5126) (width 0.4) (layer B.Cu) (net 4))
 (segment (start 131.059 114.046) (end 127.508 114.046) (width 0.25) (layer B.Cu) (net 4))
 (segment (start 139.446 112.777) (end 139.446 111.748) (width 0.25) (layer B.Cu) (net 5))
 (segment (start 139.446 111.748) (end 138.938 111.24) (width 0.25) (layer B.Cu) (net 5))
 (segment (start 138.938 111.24) (end 136.664 111.24) (width 0.25) (layer B.Cu) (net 5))
 (segment (start 136.664 111.24) (end 136.652 111.252) (width 0.25) (layer B.Cu) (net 5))
 (segment (start 136.525 113.046) (end 136.525 111.379) (width 0.25) (layer B.Cu) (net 5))
 (segment (start 136.525 111.379) (end 136.652 111.252) (width 0.25) (layer B.Cu) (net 5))
 (segment (start 139.446 116.077) (end 139.446 117.094) (width 0.25) (layer B.Cu) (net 2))
 (segment (start 135.775 117.106) (end 135.775 116.459) (width 0.25) (layer B.Cu) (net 2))
 (segment (start 136.017 117.348) (end 135.775 117.106) (width 0.25) (layer B.Cu) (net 2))
 (segment (start 139.192 117.348) (end 136.017 117.348) (width 0.25) (layer B.Cu) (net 2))
 (segment (start 139.446 117.094) (end 139.192 117.348) (width 0.25) (layer B.Cu) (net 2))
 (segment (start 135.775 116.459) (end 135.775 115.246) (width 0.25) (layer B.Cu) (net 2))
 (segment (start 135.775 115.246) (end 135.575 115.046) (width 0.25) (layer B.Cu) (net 2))
 (segment (start 140.716 108.097919) (end 140.716 115.57) (width 0.25) (layer B.Cu) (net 2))
 (segment (start 140.209 116.077) (end 139.446 116.077) (width 0.25) (layer B.Cu) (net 2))
 (segment (start 140.716 115.57) (end 140.209 116.077) (width 0.25) (layer B.Cu) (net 2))
 (segment (start 141.418919 107.395) (end 141.415119 107.3912) (width 0.25) (layer B.Cu) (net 2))
 (segment (start 142.621 107.395) (end 141.418919 107.395) (width 0.25) (layer B.Cu) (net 2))
 (segment (start 141.415119 107.3988) (end 140.716 108.097919) (width 0.25) (layer B.Cu) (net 2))
 (segment (start 141.415119 107.3912) (end 141.415119 107.3988) (width 0.25) (layer B.Cu) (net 2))
 (segment (start 133.35 113.031) (end 130.444 113.031) (width 0.25) (layer B.Cu) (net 6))
 (segment (start 130.444 113.031) (end 130.429 113.046) (width 0.25) (layer B.Cu) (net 6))
 (segment (start 134.652 111.252) (end 134.652 112.617) (width 0.25) (layer B.Cu) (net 6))
 (segment (start 134.238 113.031) (end 133.35 113.031) (width 0.25) (layer B.Cu) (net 6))
 (segment (start 134.652 112.617) (end 134.238 113.031) (width 0.25) (layer B.Cu) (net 6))
 (segment (start 134.632 109.474) (end 134.632 111.232) (width 0.25) (layer B.Cu) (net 6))
 (segment (start 134.632 111.232) (end 134.652 111.252) (width 0.25) (layer B.Cu) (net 6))
 (segment (start 133.35 116.331) (end 132.335 116.331) (width 0.25) (layer B.Cu) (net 3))
 (segment (start 129.679 117.233) (end 129.679 116.459) (width 0.25) (layer B.Cu) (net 3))
 (segment (start 129.921 117.475) (end 129.679 117.233) (width 0.25) (layer B.Cu) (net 3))
 (segment (start 131.699 117.475) (end 129.921 117.475) (width 0.25) (layer B.Cu) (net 3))
 (segment (start 132.08 117.094) (end 131.699 117.475) (width 0.25) (layer B.Cu) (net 3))
 (segment (start 132.08 116.586) (end 132.08 117.094) (width 0.25) (layer B.Cu) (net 3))
 (segment (start 132.335 116.331) (end 132.08 116.586) (width 0.25) (layer B.Cu) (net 3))
 (segment (start 129.679 116.459) (end 129.679 115.246) (width 0.25) (layer B.Cu) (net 3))
 (segment (start 129.679 115.246) (end 129.479 115.046) (width 0.25) (layer B.Cu) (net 3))
 (segment (start 141.418919 109.935) (end 142.621 109.935) (width 0.25) (layer B.Cu) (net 3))
 (segment (start 133.35 116.331) (end 134.238 116.331) (width 0.25) (layer B.Cu) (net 3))
 (segment (start 134.238 116.331) (end 135.763 117.856) (width 0.25) (layer B.Cu) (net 3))
 (segment (start 135.763 117.856) (end 139.827 117.856) (width 0.25) (layer B.Cu) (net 3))
 (segment (start 139.827 117.856) (end 141.224 116.459) (width 0.25) (layer B.Cu) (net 3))
 (segment (start 141.224 116.459) (end 141.224 110.129919) (width 0.25) (layer B.Cu) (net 3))
 (segment (start 141.224 110.129919) (end 141.418919 109.935) (width 0.25) (layer B.Cu) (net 3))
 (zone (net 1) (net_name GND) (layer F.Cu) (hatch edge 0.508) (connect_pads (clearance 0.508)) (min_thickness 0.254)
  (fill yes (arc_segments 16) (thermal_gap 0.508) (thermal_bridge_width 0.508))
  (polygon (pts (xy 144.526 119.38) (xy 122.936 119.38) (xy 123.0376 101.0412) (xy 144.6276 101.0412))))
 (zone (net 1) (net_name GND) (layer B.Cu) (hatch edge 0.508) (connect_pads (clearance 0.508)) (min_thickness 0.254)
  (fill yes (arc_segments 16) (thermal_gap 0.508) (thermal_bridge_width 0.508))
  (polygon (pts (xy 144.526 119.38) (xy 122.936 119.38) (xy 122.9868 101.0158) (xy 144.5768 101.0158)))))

